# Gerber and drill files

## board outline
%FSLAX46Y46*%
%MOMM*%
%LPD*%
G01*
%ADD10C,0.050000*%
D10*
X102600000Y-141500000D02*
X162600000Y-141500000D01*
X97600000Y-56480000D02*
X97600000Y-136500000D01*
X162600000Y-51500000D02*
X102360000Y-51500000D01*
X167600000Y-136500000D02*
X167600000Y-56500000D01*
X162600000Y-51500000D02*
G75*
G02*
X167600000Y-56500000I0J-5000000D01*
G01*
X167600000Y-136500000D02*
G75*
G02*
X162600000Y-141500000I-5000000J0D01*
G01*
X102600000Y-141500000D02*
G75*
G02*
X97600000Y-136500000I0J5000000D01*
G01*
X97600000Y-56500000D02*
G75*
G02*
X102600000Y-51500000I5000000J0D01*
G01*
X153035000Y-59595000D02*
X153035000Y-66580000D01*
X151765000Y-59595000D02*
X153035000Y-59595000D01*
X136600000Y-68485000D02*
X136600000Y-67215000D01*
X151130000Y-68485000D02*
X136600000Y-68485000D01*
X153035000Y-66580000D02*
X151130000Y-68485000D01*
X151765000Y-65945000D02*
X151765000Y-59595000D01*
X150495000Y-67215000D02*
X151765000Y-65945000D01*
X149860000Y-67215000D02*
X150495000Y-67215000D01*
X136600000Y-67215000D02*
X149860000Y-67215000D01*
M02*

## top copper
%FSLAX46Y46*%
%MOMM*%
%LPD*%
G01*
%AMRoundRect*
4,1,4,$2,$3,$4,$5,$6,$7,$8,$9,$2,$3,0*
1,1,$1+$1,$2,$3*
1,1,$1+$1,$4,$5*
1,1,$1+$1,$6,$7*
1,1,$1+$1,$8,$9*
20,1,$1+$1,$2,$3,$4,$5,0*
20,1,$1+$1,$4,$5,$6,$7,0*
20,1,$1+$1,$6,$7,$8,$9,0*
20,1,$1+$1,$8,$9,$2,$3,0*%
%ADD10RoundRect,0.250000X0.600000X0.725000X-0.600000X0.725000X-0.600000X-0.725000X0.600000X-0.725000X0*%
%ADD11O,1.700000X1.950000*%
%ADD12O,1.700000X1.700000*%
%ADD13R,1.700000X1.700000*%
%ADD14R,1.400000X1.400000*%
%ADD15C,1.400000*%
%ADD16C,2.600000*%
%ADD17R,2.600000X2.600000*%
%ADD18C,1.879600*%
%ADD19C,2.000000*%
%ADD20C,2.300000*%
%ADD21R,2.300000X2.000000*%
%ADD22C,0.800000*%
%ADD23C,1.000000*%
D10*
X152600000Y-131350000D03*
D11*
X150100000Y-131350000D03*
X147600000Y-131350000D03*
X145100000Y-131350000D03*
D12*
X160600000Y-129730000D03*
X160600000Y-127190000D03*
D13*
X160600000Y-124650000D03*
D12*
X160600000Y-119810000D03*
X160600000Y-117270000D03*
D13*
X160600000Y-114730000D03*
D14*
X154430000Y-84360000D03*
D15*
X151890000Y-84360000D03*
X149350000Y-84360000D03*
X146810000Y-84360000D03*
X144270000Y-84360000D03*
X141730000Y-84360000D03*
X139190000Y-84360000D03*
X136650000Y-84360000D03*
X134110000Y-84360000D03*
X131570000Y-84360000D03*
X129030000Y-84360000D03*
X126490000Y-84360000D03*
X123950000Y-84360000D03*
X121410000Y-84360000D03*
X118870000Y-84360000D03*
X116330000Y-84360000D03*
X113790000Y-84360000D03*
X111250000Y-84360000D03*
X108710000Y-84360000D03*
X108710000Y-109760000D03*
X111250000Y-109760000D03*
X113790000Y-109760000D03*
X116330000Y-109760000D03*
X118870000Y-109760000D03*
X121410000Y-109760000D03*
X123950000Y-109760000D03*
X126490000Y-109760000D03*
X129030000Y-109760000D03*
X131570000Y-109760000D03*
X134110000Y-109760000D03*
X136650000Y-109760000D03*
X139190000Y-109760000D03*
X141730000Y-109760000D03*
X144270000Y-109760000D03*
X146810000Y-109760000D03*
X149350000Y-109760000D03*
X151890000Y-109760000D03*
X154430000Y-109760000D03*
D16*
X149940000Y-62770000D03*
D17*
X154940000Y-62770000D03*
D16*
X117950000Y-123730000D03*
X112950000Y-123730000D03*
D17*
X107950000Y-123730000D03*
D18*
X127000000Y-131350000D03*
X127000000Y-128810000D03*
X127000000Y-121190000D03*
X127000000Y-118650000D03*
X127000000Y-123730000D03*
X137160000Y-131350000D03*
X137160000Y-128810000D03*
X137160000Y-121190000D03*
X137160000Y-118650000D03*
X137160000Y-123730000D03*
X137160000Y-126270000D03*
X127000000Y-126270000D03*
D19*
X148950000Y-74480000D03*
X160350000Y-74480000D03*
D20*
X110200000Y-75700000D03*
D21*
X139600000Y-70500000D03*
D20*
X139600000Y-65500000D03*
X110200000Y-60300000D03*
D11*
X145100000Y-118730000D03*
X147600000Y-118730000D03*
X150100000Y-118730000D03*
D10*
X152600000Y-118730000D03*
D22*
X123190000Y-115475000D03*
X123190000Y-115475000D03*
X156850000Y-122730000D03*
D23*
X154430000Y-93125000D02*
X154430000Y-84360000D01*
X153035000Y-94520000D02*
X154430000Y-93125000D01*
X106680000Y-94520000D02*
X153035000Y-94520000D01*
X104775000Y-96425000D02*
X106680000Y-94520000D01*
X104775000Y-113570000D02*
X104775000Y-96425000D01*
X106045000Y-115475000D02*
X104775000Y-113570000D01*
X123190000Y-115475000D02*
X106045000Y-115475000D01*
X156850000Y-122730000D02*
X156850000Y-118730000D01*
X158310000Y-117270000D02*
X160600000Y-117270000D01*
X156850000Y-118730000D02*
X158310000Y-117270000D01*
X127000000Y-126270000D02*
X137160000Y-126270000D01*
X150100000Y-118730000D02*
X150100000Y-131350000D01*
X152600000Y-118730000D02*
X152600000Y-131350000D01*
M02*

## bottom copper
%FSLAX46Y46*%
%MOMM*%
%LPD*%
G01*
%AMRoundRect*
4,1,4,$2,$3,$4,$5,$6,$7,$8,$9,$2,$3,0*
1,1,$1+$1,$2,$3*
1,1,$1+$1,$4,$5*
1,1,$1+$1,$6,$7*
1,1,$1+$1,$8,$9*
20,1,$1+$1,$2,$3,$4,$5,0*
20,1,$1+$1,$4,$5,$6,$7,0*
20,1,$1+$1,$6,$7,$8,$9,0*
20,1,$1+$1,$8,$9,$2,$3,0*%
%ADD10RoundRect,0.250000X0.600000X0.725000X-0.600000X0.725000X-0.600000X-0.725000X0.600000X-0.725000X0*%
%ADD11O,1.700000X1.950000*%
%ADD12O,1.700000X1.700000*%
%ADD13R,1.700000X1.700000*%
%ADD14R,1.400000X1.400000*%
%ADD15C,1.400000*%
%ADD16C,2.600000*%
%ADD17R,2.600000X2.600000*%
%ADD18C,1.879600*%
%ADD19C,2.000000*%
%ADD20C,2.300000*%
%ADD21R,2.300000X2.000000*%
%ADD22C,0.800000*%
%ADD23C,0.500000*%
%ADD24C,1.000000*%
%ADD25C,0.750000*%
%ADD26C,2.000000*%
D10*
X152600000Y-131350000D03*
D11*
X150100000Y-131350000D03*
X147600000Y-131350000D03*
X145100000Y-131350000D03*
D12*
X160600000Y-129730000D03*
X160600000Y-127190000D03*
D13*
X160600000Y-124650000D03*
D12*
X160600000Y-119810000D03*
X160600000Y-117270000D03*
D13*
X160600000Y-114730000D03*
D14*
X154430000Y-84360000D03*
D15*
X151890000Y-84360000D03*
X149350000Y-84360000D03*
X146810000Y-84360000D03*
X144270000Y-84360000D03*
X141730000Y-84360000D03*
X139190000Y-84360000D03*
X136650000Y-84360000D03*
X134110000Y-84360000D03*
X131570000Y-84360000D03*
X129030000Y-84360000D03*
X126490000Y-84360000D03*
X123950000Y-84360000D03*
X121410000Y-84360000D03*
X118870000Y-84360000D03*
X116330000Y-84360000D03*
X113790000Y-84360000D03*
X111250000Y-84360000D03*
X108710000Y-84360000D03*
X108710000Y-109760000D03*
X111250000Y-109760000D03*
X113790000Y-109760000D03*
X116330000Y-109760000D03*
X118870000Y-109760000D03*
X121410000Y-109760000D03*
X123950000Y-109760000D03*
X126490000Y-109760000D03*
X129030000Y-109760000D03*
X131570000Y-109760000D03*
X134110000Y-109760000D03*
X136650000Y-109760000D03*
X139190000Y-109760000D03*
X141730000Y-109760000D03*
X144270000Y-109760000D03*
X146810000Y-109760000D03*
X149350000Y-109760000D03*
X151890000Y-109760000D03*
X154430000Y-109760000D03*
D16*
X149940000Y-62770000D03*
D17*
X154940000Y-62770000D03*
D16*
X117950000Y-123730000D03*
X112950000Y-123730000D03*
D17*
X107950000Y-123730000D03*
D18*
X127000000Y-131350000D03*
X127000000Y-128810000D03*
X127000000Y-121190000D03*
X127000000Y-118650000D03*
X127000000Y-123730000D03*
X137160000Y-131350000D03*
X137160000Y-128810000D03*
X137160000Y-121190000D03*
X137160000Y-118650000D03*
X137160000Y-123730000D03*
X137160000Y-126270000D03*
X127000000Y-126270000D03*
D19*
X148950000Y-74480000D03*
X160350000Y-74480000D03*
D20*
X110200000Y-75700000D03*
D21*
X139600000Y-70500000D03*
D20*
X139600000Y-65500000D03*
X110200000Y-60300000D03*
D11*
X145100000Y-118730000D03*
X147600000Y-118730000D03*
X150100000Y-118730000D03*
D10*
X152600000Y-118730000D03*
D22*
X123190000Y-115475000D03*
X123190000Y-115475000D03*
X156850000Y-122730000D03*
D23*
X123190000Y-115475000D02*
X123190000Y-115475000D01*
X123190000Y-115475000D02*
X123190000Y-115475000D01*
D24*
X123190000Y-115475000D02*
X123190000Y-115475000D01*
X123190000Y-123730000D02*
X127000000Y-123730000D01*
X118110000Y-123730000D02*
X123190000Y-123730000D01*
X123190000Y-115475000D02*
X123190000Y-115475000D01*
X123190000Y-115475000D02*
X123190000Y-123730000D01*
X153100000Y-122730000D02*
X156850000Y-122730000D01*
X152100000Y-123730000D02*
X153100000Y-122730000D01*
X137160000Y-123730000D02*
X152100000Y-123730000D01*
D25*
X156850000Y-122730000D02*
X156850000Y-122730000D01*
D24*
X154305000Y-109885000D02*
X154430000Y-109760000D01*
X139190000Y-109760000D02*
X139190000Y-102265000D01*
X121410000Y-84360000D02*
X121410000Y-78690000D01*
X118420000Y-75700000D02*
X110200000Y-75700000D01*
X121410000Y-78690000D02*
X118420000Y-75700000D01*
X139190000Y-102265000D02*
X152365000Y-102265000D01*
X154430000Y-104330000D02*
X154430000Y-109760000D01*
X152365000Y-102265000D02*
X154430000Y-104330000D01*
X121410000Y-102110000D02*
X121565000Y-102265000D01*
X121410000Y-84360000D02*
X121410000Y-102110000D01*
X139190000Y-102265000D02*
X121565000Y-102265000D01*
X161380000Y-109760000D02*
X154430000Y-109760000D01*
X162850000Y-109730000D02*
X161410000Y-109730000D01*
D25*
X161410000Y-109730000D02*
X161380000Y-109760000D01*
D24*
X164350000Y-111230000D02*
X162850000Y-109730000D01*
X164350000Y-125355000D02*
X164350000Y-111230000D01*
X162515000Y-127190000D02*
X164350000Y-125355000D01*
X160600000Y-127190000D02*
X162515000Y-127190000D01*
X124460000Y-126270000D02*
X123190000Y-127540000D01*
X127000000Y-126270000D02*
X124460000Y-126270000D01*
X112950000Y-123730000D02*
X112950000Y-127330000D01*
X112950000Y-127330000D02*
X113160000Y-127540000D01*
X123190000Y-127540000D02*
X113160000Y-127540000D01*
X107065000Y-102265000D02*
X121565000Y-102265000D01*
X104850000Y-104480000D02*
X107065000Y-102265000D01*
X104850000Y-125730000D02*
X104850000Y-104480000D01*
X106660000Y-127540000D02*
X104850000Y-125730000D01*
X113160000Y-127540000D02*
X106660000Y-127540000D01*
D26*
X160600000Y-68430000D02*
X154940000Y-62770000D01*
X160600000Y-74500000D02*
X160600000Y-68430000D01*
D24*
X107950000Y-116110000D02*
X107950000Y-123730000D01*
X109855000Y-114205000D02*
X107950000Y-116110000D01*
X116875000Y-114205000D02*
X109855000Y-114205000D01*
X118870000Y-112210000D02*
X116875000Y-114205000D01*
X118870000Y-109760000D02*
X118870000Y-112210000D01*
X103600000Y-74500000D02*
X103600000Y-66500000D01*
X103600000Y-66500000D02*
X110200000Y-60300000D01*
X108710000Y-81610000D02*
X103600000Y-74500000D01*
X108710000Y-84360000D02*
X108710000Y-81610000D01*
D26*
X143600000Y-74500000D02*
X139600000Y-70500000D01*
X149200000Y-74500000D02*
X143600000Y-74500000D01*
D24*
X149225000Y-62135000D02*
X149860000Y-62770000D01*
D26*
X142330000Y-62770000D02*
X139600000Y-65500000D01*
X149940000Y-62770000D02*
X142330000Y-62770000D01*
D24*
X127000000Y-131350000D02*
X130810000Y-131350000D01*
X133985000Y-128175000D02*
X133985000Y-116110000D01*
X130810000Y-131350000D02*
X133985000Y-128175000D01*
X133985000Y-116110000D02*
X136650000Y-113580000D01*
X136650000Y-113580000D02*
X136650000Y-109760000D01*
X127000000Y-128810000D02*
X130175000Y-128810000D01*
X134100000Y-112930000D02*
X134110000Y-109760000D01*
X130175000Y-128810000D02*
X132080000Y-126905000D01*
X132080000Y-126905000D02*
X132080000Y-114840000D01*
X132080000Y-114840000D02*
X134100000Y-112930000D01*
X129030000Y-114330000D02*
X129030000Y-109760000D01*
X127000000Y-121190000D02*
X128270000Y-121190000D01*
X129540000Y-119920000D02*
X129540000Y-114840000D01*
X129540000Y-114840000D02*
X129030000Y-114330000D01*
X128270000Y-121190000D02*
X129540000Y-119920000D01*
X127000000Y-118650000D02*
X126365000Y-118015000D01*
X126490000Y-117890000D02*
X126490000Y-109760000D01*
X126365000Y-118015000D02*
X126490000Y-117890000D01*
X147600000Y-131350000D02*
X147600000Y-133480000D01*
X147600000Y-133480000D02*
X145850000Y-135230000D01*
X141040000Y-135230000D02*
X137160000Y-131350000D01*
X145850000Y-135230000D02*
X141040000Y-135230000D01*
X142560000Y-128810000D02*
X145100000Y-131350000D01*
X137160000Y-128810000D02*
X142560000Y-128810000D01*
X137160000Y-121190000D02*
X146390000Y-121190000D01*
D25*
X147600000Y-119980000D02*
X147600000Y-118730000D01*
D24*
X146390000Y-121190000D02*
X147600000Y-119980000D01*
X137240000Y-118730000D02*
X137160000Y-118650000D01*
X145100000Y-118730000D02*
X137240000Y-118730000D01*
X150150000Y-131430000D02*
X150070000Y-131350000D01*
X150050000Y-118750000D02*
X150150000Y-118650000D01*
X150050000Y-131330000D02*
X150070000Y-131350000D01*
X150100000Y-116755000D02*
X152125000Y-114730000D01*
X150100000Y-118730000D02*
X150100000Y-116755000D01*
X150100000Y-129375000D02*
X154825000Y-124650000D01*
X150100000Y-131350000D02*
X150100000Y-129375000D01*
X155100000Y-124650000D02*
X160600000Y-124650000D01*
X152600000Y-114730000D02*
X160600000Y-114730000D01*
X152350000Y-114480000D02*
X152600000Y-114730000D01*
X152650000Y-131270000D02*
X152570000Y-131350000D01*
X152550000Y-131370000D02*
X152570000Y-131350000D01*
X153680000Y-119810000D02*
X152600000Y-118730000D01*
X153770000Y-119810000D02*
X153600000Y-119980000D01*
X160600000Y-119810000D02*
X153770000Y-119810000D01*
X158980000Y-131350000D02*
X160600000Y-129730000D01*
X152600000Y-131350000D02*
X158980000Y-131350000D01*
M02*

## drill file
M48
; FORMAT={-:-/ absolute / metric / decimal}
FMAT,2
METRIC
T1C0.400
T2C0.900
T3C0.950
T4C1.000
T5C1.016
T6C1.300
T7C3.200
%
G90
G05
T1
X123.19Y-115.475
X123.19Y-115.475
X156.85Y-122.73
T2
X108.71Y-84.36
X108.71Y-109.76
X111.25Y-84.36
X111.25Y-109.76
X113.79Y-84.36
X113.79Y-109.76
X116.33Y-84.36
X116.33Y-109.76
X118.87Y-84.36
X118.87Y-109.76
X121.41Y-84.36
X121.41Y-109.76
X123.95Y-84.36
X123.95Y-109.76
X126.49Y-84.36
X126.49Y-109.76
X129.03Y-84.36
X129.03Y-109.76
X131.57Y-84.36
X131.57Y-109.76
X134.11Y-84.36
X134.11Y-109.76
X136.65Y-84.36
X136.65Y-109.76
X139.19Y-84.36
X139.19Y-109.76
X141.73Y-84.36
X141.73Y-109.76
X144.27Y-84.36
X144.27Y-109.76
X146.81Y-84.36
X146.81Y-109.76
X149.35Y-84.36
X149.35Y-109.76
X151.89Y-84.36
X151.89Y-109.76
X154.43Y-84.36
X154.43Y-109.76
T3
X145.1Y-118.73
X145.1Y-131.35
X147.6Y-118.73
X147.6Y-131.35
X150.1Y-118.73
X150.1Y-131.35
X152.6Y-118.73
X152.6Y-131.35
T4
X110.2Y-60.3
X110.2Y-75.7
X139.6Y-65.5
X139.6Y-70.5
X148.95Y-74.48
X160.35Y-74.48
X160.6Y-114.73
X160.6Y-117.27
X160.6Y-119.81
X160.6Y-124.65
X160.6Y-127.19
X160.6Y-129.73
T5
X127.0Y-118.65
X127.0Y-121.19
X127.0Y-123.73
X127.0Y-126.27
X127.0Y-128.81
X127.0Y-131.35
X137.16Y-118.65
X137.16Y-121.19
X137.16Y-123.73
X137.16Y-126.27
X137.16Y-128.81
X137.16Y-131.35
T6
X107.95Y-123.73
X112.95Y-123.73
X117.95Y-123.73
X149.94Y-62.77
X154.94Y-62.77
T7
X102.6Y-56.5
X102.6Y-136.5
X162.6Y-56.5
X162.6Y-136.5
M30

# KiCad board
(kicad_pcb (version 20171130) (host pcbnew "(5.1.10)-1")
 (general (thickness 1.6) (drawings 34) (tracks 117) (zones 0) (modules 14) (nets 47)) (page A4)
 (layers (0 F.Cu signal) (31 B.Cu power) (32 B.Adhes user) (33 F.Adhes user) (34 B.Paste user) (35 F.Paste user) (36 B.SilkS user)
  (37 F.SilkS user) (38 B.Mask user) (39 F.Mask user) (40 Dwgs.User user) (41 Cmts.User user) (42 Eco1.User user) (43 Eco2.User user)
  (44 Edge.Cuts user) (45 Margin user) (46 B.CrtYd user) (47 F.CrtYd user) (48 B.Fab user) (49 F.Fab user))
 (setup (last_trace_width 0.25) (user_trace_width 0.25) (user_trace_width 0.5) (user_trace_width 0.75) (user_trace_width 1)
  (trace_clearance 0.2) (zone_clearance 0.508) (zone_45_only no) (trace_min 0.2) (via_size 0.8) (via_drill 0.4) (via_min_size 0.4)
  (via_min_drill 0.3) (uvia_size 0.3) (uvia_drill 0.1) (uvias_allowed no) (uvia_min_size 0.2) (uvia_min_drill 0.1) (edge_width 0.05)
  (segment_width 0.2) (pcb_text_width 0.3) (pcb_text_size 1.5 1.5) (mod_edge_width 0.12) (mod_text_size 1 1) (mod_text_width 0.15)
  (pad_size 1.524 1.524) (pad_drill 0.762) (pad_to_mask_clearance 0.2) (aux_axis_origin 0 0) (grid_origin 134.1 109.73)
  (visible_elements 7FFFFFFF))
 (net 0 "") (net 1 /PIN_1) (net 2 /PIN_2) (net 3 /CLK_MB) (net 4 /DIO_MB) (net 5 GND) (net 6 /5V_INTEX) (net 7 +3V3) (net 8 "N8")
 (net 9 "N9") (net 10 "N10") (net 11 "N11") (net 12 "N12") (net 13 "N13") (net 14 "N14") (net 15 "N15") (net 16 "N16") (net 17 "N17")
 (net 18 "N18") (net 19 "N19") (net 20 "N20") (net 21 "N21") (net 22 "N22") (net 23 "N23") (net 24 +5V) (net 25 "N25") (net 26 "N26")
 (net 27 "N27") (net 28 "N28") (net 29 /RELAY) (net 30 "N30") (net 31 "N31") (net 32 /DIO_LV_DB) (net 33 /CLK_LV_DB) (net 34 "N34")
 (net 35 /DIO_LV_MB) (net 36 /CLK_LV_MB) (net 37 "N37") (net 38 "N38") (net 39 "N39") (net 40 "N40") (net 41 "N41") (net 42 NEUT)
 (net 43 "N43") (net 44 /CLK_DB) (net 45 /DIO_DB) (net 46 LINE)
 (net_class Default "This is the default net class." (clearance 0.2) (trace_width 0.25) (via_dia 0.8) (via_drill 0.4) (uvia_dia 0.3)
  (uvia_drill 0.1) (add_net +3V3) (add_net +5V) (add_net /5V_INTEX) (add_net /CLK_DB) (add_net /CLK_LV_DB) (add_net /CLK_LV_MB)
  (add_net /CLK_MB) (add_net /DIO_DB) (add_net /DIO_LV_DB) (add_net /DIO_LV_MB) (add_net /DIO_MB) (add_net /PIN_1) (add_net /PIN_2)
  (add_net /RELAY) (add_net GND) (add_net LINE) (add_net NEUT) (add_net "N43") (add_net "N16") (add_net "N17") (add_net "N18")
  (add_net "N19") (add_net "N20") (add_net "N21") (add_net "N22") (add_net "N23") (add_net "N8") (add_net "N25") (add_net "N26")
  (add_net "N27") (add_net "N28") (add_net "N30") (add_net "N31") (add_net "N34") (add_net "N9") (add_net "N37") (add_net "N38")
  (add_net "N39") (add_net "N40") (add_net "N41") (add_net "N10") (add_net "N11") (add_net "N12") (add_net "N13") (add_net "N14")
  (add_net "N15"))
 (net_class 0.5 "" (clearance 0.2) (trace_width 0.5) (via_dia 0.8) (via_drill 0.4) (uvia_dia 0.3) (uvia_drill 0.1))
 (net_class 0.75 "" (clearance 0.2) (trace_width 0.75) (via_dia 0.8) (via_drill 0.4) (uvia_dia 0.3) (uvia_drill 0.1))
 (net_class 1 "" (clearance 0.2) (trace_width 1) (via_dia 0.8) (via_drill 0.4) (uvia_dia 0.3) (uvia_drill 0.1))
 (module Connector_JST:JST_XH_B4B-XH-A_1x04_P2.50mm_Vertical (layer F.Cu) (at 152.6 131.35 180)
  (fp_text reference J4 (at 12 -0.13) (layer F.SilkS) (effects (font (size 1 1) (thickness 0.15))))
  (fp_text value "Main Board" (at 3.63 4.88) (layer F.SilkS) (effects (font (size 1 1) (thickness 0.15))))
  (pad 1 thru_hole roundrect (at 0 0 180) (size 1.7 1.95) (drill 0.95) (layers *.Cu *.Mask) (roundrect_rratio 0.1470588235294118)
   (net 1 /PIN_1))
  (pad 2 thru_hole oval (at 2.5 0 180) (size 1.7 1.95) (drill 0.95) (layers *.Cu *.Mask) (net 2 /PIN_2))
  (pad 3 thru_hole oval (at 5 0 180) (size 1.7 1.95) (drill 0.95) (layers *.Cu *.Mask) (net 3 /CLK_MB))
  (pad 4 thru_hole oval (at 7.5 0 180) (size 1.7 1.95) (drill 0.95) (layers *.Cu *.Mask) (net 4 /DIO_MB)))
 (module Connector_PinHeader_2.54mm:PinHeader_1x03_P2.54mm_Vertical (layer F.Cu) (at 160.6 124.65)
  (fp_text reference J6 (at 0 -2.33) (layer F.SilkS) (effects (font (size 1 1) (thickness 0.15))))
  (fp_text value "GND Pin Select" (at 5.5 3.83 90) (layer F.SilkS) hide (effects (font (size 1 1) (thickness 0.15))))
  (pad 3 thru_hole oval (at 0 5.08) (size 1.7 1.7) (drill 1) (layers *.Cu *.Mask) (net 1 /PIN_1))
  (pad 2 thru_hole oval (at 0 2.54) (size 1.7 1.7) (drill 1) (layers *.Cu *.Mask) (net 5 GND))
  (pad 1 thru_hole rect (at 0 0) (size 1.7 1.7) (drill 1) (layers *.Cu *.Mask) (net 2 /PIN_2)))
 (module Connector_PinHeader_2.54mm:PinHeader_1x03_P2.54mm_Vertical (layer F.Cu) (at 160.6 114.73)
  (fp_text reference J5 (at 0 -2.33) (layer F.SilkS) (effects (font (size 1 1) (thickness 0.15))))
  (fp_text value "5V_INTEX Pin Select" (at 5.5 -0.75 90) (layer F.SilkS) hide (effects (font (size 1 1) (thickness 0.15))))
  (pad 3 thru_hole oval (at 0 5.08) (size 1.7 1.7) (drill 1) (layers *.Cu *.Mask) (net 1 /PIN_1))
  (pad 2 thru_hole oval (at 0 2.54) (size 1.7 1.7) (drill 1) (layers *.Cu *.Mask) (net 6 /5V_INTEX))
  (pad 1 thru_hole rect (at 0 0) (size 1.7 1.7) (drill 1) (layers *.Cu *.Mask) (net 2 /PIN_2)))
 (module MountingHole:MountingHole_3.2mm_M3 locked (layer F.Cu) (at 162.6 136.5)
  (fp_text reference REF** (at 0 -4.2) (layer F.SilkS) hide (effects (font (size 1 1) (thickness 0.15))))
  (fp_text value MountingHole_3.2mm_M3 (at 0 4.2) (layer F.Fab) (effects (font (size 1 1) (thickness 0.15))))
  (pad 1 np_thru_hole circle (at 0 0) (size 3.2 3.2) (drill 3.2) (layers *.Cu *.Mask)))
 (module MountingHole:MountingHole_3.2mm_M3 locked (layer F.Cu) (at 102.6 136.5)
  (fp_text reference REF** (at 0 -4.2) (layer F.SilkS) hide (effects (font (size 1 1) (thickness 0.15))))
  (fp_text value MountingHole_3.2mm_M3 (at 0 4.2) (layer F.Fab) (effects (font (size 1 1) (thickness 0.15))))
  (pad 1 np_thru_hole circle (at 0 0) (size 3.2 3.2) (drill 3.2) (layers *.Cu *.Mask)))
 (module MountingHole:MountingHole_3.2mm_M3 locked (layer F.Cu) (at 162.6 56.5)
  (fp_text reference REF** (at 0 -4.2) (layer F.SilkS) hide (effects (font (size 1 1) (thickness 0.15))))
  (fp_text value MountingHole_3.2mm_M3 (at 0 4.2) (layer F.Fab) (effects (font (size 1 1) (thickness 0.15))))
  (pad 1 np_thru_hole circle (at 0 0) (size 3.2 3.2) (drill 3.2) (layers *.Cu *.Mask)))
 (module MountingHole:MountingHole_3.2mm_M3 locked (layer F.Cu) (at 102.6 56.5)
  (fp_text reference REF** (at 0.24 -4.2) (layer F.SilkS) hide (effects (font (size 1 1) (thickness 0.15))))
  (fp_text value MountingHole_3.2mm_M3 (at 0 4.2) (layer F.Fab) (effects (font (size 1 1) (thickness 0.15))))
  (pad 1 np_thru_hole circle (at 0 0) (size 3.2 3.2) (drill 3.2) (layers *.Cu *.Mask)))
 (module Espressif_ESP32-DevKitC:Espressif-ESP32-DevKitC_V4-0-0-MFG (layer F.Cu) (at 134.62 97.06 270)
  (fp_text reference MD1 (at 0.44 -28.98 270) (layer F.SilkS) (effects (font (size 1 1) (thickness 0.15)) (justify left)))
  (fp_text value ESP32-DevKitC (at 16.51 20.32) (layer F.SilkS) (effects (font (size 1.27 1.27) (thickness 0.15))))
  (pad 1 thru_hole rect (at -12.7 -19.81 270) (size 1.4 1.4) (drill 0.9) (layers *.Cu *.Paste *.Mask) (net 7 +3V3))
  (pad 2 thru_hole circle (at -12.7 -17.27 270) (size 1.4 1.4) (drill 0.9) (layers *.Cu *.Paste *.Mask) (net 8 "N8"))
  (pad 3 thru_hole circle (at -12.7 -14.73 270) (size 1.4 1.4) (drill 0.9) (layers *.Cu *.Paste *.Mask) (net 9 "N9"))
  (pad 4 thru_hole circle (at -12.7 -12.19 270) (size 1.4 1.4) (drill 0.9) (layers *.Cu *.Paste *.Mask) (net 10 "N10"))
  (pad 5 thru_hole circle (at -12.7 -9.65 270) (size 1.4 1.4) (drill 0.9) (layers *.Cu *.Paste *.Mask) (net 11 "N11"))
  (pad 6 thru_hole circle (at -12.7 -7.11 270) (size 1.4 1.4) (drill 0.9) (layers *.Cu *.Paste *.Mask) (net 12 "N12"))
  (pad 7 thru_hole circle (at -12.7 -4.57 270) (size 1.4 1.4) (drill 0.9) (layers *.Cu *.Paste *.Mask) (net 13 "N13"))
  (pad 8 thru_hole circle (at -12.7 -2.03 270) (size 1.4 1.4) (drill 0.9) (layers *.Cu *.Paste *.Mask) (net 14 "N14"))
  (pad 9 thru_hole circle (at -12.7 0.51 270) (size 1.4 1.4) (drill 0.9) (layers *.Cu *.Paste *.Mask) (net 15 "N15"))
  (pad 10 thru_hole circle (at -12.7 3.05 270) (size 1.4 1.4) (drill 0.9) (layers *.Cu *.Paste *.Mask) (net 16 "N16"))
  (pad 11 thru_hole circle (at -12.7 5.59 270) (size 1.4 1.4) (drill 0.9) (layers *.Cu *.Paste *.Mask) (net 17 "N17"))
  (pad 12 thru_hole circle (at -12.7 8.13 270) (size 1.4 1.4) (drill 0.9) (layers *.Cu *.Paste *.Mask) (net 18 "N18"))
  (pad 13 thru_hole circle (at -12.7 10.67 270) (size 1.4 1.4) (drill 0.9) (layers *.Cu *.Paste *.Mask) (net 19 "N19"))
  (pad 14 thru_hole circle (at -12.7 13.21 270) (size 1.4 1.4) (drill 0.9) (layers *.Cu *.Paste *.Mask) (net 5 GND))
  (pad 15 thru_hole circle (at -12.7 15.75 270) (size 1.4 1.4) (drill 0.9) (layers *.Cu *.Paste *.Mask) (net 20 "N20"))
  (pad 16 thru_hole circle (at -12.7 18.29 270) (size 1.4 1.4) (drill 0.9) (layers *.Cu *.Paste *.Mask) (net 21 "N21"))
  (pad 17 thru_hole circle (at -12.7 20.83 270) (size 1.4 1.4) (drill 0.9) (layers *.Cu *.Paste *.Mask) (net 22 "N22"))
  (pad 18 thru_hole circle (at -12.7 23.37 270) (size 1.4 1.4) (drill 0.9) (layers *.Cu *.Paste *.Mask) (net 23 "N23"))
  (pad 19 thru_hole circle (at -12.7 25.91 270) (size 1.4 1.4) (drill 0.9) (layers *.Cu *.Paste *.Mask) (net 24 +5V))
  (pad 20 thru_hole circle (at 12.7 25.91 270) (size 1.4 1.4) (drill 0.9) (layers *.Cu *.Paste *.Mask) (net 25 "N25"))
  (pad 21 thru_hole circle (at 12.7 23.37 270) (size 1.4 1.4) (drill 0.9) (layers *.Cu *.Paste *.Mask) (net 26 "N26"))
  (pad 22 thru_hole circle (at 12.7 20.83 270) (size 1.4 1.4) (drill 0.9) (layers *.Cu *.Paste *.Mask) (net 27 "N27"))
  (pad 23 thru_hole circle (at 12.7 18.29 270) (size 1.4 1.4) (drill 0.9) (layers *.Cu *.Paste *.Mask) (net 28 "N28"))
  (pad 24 thru_hole circle (at 12.7 15.75 270) (size 1.4 1.4) (drill 0.9) (layers *.Cu *.Paste *.Mask) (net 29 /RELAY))
  (pad 25 thru_hole circle (at 12.7 13.21 270) (size 1.4 1.4) (drill 0.9) (layers *.Cu *.Paste *.Mask) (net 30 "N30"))
  (pad 26 thru_hole circle (at 12.7 10.67 270) (size 1.4 1.4) (drill 0.9) (layers *.Cu *.Paste *.Mask) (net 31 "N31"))
  (pad 27 thru_hole circle (at 12.7 8.13 270) (size 1.4 1.4) (drill 0.9) (layers *.Cu *.Paste *.Mask) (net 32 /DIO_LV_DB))
  (pad 28 thru_hole circle (at 12.7 5.59 270) (size 1.4 1.4) (drill 0.9) (layers *.Cu *.Paste *.Mask) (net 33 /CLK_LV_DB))
  (pad 29 thru_hole circle (at 12.7 3.05 270) (size 1.4 1.4) (drill 0.9) (layers *.Cu *.Paste *.Mask) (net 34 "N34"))
  (pad 30 thru_hole circle (at 12.7 0.51 270) (size 1.4 1.4) (drill 0.9) (layers *.Cu *.Paste *.Mask) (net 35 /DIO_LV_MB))
  (pad 31 thru_hole circle (at 12.7 -2.03 270) (size 1.4 1.4) (drill 0.9) (layers *.Cu *.Paste *.Mask) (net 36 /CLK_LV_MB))
  (pad 32 thru_hole circle (at 12.7 -4.57 270) (size 1.4 1.4) (drill 0.9) (layers *.Cu *.Paste *.Mask) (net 5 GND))
  (pad 33 thru_hole circle (at 12.7 -7.11 270) (size 1.4 1.4) (drill 0.9) (layers *.Cu *.Paste *.Mask) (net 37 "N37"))
  (pad 34 thru_hole circle (at 12.7 -9.65 270) (size 1.4 1.4) (drill 0.9) (layers *.Cu *.Paste *.Mask) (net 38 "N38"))
  (pad 35 thru_hole circle (at 12.7 -12.19 270) (size 1.4 1.4) (drill 0.9) (layers *.Cu *.Paste *.Mask) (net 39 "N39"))
  (pad 36 thru_hole circle (at 12.7 -14.73 270) (size 1.4 1.4) (drill 0.9) (layers *.Cu *.Paste *.Mask) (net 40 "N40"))
  (pad 37 thru_hole circle (at 12.7 -17.27 270) (size 1.4 1.4) (drill 0.9) (layers *.Cu *.Paste *.Mask) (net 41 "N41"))
  (pad 38 thru_hole circle (at 12.7 -19.81 270) (size 1.4 1.4) (drill 0.9) (layers *.Cu *.Paste *.Mask) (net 5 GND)))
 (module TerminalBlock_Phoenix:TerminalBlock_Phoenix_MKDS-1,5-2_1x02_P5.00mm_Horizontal (layer F.Cu) (at 154.94 62.77 180)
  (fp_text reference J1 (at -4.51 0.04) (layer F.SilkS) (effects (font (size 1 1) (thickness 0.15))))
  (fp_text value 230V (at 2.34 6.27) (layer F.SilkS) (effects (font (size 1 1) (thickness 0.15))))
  (pad 2 thru_hole circle (at 5 0 180) (size 2.6 2.6) (drill 1.3) (layers *.Cu *.Mask) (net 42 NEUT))
  (pad 1 thru_hole rect (at 0 0 180) (size 2.6 2.6) (drill 1.3) (layers *.Cu *.Mask) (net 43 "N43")))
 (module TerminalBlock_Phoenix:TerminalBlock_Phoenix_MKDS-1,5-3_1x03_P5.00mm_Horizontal (layer F.Cu) (at 107.95 123.73)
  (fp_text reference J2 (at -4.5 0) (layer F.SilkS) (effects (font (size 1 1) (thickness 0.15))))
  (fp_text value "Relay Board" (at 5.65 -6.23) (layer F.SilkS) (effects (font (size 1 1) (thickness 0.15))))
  (pad 3 thru_hole circle (at 10 0) (size 2.6 2.6) (drill 1.3) (layers *.Cu *.Mask) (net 7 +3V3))
  (pad 2 thru_hole circle (at 5 0) (size 2.6 2.6) (drill 1.3) (layers *.Cu *.Mask) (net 5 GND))
  (pad 1 thru_hole rect (at 0 0) (size 2.6 2.6) (drill 1.3) (layers *.Cu *.Mask) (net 29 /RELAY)))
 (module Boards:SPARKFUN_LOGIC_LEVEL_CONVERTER (layer F.Cu) (at 132.08 125)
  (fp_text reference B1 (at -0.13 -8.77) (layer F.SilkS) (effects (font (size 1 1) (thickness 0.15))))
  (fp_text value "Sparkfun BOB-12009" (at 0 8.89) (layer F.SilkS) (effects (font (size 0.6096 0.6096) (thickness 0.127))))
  (pad LV4 thru_hole circle (at -5.08 6.35) (size 1.8796 1.8796) (drill 1.016) (layers *.Cu *.Mask) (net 36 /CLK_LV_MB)
   (solder_mask_margin 0.1016))
  (pad LV3 thru_hole circle (at -5.08 3.81) (size 1.8796 1.8796) (drill 1.016) (layers *.Cu *.Mask) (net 35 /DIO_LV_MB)
   (solder_mask_margin 0.1016))
  (pad LV2 thru_hole circle (at -5.08 -3.81) (size 1.8796 1.8796) (drill 1.016) (layers *.Cu *.Mask) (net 33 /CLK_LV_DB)
   (solder_mask_margin 0.1016))
  (pad LV1 thru_hole circle (at -5.08 -6.35) (size 1.8796 1.8796) (drill 1.016) (layers *.Cu *.Mask) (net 32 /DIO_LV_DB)
   (solder_mask_margin 0.1016))
  (pad LV thru_hole circle (at -5.08 -1.27) (size 1.8796 1.8796) (drill 1.016) (layers *.Cu *.Mask) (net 7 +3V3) (solder_mask_margin 0.1016))
  (pad HV4 thru_hole circle (at 5.08 6.35) (size 1.8796 1.8796) (drill 1.016) (layers *.Cu *.Mask) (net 3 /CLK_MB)
   (solder_mask_margin 0.1016))
  (pad HV3 thru_hole circle (at 5.08 3.81) (size 1.8796 1.8796) (drill 1.016) (layers *.Cu *.Mask) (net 4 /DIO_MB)
   (solder_mask_margin 0.1016))
  (pad HV2 thru_hole circle (at 5.08 -3.81) (size 1.8796 1.8796) (drill 1.016) (layers *.Cu *.Mask) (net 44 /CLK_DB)
   (solder_mask_margin 0.1016))
  (pad HV1 thru_hole circle (at 5.08 -6.35) (size 1.8796 1.8796) (drill 1.016) (layers *.Cu *.Mask) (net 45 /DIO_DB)
   (solder_mask_margin 0.1016))
  (pad HV thru_hole circle (at 5.08 -1.27) (size 1.8796 1.8796) (drill 1.016) (layers *.Cu *.Mask) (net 6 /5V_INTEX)
   (solder_mask_margin 0.1016))
  (pad GND2 thru_hole circle (at 5.08 1.27) (size 1.8796 1.8796) (drill 1.016) (layers *.Cu *.Mask) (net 5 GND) (solder_mask_margin 0.1016))
  (pad GND1 thru_hole circle (at -5.08 1.27) (size 1.8796 1.8796) (drill 1.016) (layers *.Cu *.Mask) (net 5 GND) (solder_mask_margin 0.1016)))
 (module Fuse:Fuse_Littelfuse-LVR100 (layer F.Cu) (at 160.35 74.48 180)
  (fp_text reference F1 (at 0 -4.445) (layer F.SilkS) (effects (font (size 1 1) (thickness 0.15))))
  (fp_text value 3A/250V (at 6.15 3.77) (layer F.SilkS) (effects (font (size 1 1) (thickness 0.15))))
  (pad 2 thru_hole circle (at 11.4 0 180) (size 2 2) (drill 1) (layers *.Cu *.Mask) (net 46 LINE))
  (pad 1 thru_hole circle (at 0 0 180) (size 2 2) (drill 1) (layers *.Cu *.Mask) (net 43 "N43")))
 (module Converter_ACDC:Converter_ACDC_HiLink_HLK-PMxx (layer F.Cu) (at 139.6 70.5 180)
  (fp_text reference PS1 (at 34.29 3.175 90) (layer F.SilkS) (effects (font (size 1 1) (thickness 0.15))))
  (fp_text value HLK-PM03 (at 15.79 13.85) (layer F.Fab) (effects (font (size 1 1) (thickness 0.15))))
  (pad 3 thru_hole circle (at 29.4 -5.2 180) (size 2.3 2.3) (drill 1) (layers *.Cu *.Mask) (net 5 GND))
  (pad 1 thru_hole rect (at 0 0 180) (size 2.3 2) (drill 1) (layers *.Cu *.Mask) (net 46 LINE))
  (pad 2 thru_hole circle (at 0 5 180) (size 2.3 2.3) (drill 1) (layers *.Cu *.Mask) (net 42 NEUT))
  (pad 4 thru_hole circle (at 29.4 10.2 180) (size 2.3 2.3) (drill 1) (layers *.Cu *.Mask) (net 24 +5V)))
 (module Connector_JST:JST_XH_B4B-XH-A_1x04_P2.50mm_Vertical (layer F.Cu) (at 152.6 118.73 180)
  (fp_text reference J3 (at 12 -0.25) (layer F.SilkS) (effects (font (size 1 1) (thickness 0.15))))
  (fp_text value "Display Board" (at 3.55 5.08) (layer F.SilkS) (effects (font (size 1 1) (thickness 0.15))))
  (pad 4 thru_hole oval (at 7.5 0 180) (size 1.7 1.95) (drill 0.95) (layers *.Cu *.Mask) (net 45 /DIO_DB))
  (pad 3 thru_hole oval (at 5 0 180) (size 1.7 1.95) (drill 0.95) (layers *.Cu *.Mask) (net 44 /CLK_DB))
  (pad 2 thru_hole oval (at 2.5 0 180) (size 1.7 1.95) (drill 0.95) (layers *.Cu *.Mask) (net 2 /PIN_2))
  (pad 1 thru_hole roundrect (at 0 0 180) (size 1.7 1.95) (drill 0.95) (layers *.Cu *.Mask) (roundrect_rratio 0.1470588235294118)
   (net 1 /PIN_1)))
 (gr_line (start 102.6 141.5) (end 162.6 141.5) (layer Edge.Cuts) (width 0.05))
 (gr_line (start 97.6 56.48) (end 97.6 136.5) (layer Edge.Cuts) (width 0.05))
 (gr_line (start 162.6 51.5) (end 102.36 51.5) (layer Edge.Cuts) (width 0.05))
 (gr_line (start 167.6 136.5) (end 167.6 56.5) (layer Edge.Cuts) (width 0.05))
 (gr_arc (start 162.6 56.5) (end 167.6 56.5) (angle -90) (layer Edge.Cuts) (width 0.05))
 (gr_arc (start 162.6 136.5) (end 162.6 141.5) (angle -90) (layer Edge.Cuts) (width 0.05))
 (gr_arc (start 102.6 136.5) (end 97.6 136.5) (angle -90) (layer Edge.Cuts) (width 0.05))
 (gr_arc (start 102.6 56.5) (end 102.6 51.5) (angle -90) (layer Edge.Cuts) (width 0.05))
 (gr_line (start 153.035 59.595) (end 153.035 66.58) (layer Edge.Cuts) (width 0.05))
 (gr_line (start 151.765 59.595) (end 153.035 59.595) (layer Edge.Cuts) (width 0.05))
 (gr_line (start 136.6 68.485) (end 136.6 67.215) (layer Edge.Cuts) (width 0.05))
 (gr_line (start 151.13 68.485) (end 136.6 68.485) (layer Edge.Cuts) (width 0.05))
 (gr_line (start 153.035 66.58) (end 151.13 68.485) (layer Edge.Cuts) (width 0.05))
 (gr_line (start 151.765 65.945) (end 151.765 59.595) (layer Edge.Cuts) (width 0.05))
 (gr_line (start 150.495 67.215) (end 151.765 65.945) (layer Edge.Cuts) (width 0.05))
 (gr_line (start 149.86 67.215) (end 150.495 67.215) (layer Edge.Cuts) (width 0.05))
 (gr_line (start 136.6 67.215) (end 149.86 67.215) (layer Edge.Cuts) (width 0.05))
 (segment (start 123.19 115.475) (end 123.19 115.475) (width 0.5) (layer B.Cu) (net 7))
 (segment (start 123.19 115.475) (end 123.19 115.475) (width 0.5) (layer B.Cu) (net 7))
 (segment (start 123.19 115.475) (end 123.19 115.475) (width 1) (layer B.Cu) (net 7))
 (segment (start 123.19 123.73) (end 127 123.73) (width 1) (layer B.Cu) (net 7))
 (segment (start 118.11 123.73) (end 123.19 123.73) (width 1) (layer B.Cu) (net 7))
 (segment (start 123.19 115.475) (end 123.19 115.475) (width 1) (layer B.Cu) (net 7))
 (via (at 123.19 115.475) (size 0.8) (drill 0.4) (layers F.Cu B.Cu) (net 7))
 (segment (start 123.19 115.475) (end 123.19 123.73) (width 1) (layer B.Cu) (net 7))
 (via (at 123.19 115.475) (size 0.8) (drill 0.4) (layers F.Cu B.Cu) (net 7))
 (segment (start 154.43 93.125) (end 154.43 84.36) (width 1) (layer F.Cu) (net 7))
 (segment (start 153.035 94.52) (end 154.43 93.125) (width 1) (layer F.Cu) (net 7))
 (segment (start 106.68 94.52) (end 153.035 94.52) (width 1) (layer F.Cu) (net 7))
 (segment (start 104.775 96.425) (end 106.68 94.52) (width 1) (layer F.Cu) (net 7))
 (segment (start 104.775 113.57) (end 104.775 96.425) (width 1) (layer F.Cu) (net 7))
 (segment (start 106.045 115.475) (end 104.775 113.57) (width 1) (layer F.Cu) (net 7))
 (segment (start 123.19 115.475) (end 106.045 115.475) (width 1) (layer F.Cu) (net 7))
 (segment (start 153.1 122.73) (end 156.85 122.73) (width 1) (layer B.Cu) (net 6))
 (segment (start 152.1 123.73) (end 153.1 122.73) (width 1) (layer B.Cu) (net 6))
 (segment (start 137.16 123.73) (end 152.1 123.73) (width 1) (layer B.Cu) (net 6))
 (segment (start 156.85 122.73) (end 156.85 122.73) (width 0.75) (layer B.Cu) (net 6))
 (via (at 156.85 122.73) (size 0.8) (drill 0.4) (layers F.Cu B.Cu) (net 6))
 (segment (start 156.85 122.73) (end 156.85 118.73) (width 1) (layer F.Cu) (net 6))
 (segment (start 158.31 117.27) (end 160.6 117.27) (width 1) (layer F.Cu) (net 6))
 (segment (start 156.85 118.73) (end 158.31 117.27) (width 1) (layer F.Cu) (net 6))
 (segment (start 154.305 109.885) (end 154.43 109.76) (width 1) (layer B.Cu) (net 5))
 (segment (start 139.19 109.76) (end 139.19 102.265) (width 1) (layer B.Cu) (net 5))
 (segment (start 121.41 84.36) (end 121.41 78.69) (width 1) (layer B.Cu) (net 5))
 (segment (start 118.42 75.7) (end 110.2 75.7) (width 1) (layer B.Cu) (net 5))
 (segment (start 121.41 78.69) (end 118.42 75.7) (width 1) (layer B.Cu) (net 5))
 (segment (start 139.19 102.265) (end 152.365 102.265) (width 1) (layer B.Cu) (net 5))
 (segment (start 154.43 104.33) (end 154.43 109.76) (width 1) (layer B.Cu) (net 5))
 (segment (start 152.365 102.265) (end 154.43 104.33) (width 1) (layer B.Cu) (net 5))
 (segment (start 121.41 102.11) (end 121.565 102.265) (width 1) (layer B.Cu) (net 5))
 (segment (start 121.41 84.36) (end 121.41 102.11) (width 1) (layer B.Cu) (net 5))
 (segment (start 139.19 102.265) (end 121.565 102.265) (width 1) (layer B.Cu) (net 5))
 (segment (start 127 126.27) (end 137.16 126.27) (width 1) (layer F.Cu) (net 5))
 (segment (start 161.38 109.76) (end 154.43 109.76) (width 1) (layer B.Cu) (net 5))
 (segment (start 162.85 109.73) (end 161.41 109.73) (width 1) (layer B.Cu) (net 5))
 (segment (start 161.41 109.73) (end 161.38 109.76) (width 0.75) (layer B.Cu) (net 5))
 (segment (start 164.35 111.23) (end 162.85 109.73) (width 1) (layer B.Cu) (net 5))
 (segment (start 164.35 125.355) (end 164.35 111.23) (width 1) (layer B.Cu) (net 5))
 (segment (start 162.515 127.19) (end 164.35 125.355) (width 1) (layer B.Cu) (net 5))
 (segment (start 160.6 127.19) (end 162.515 127.19) (width 1) (layer B.Cu) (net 5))
 (segment (start 124.46 126.27) (end 123.19 127.54) (width 1) (layer B.Cu) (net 5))
 (segment (start 127 126.27) (end 124.46 126.27) (width 1) (layer B.Cu) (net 5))
 (segment (start 112.95 123.73) (end 112.95 127.33) (width 1) (layer B.Cu) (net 5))
 (segment (start 112.95 127.33) (end 113.16 127.54) (width 1) (layer B.Cu) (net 5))
 (segment (start 123.19 127.54) (end 113.16 127.54) (width 1) (layer B.Cu) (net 5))
 (segment (start 107.065 102.265) (end 121.565 102.265) (width 1) (layer B.Cu) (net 5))
 (segment (start 104.85 104.48) (end 107.065 102.265) (width 1) (layer B.Cu) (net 5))
 (segment (start 104.85 125.73) (end 104.85 104.48) (width 1) (layer B.Cu) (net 5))
 (segment (start 106.66 127.54) (end 104.85 125.73) (width 1) (layer B.Cu) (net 5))
 (segment (start 113.16 127.54) (end 106.66 127.54) (width 1) (layer B.Cu) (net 5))
 (segment (start 160.6 68.43) (end 154.94 62.77) (width 2) (layer B.Cu) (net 43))
 (segment (start 160.6 74.5) (end 160.6 68.43) (width 2) (layer B.Cu) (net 43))
 (segment (start 107.95 116.11) (end 107.95 123.73) (width 1) (layer B.Cu) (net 29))
 (segment (start 109.855 114.205) (end 107.95 116.11) (width 1) (layer B.Cu) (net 29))
 (segment (start 116.875 114.205) (end 109.855 114.205) (width 1) (layer B.Cu) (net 29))
 (segment (start 118.87 112.21) (end 116.875 114.205) (width 1) (layer B.Cu) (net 29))
 (segment (start 118.87 109.76) (end 118.87 112.21) (width 1) (layer B.Cu) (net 29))
 (segment (start 103.6 74.5) (end 103.6 66.5) (width 1) (layer B.Cu) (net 24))
 (segment (start 103.6 66.5) (end 110.2 60.3) (width 1) (layer B.Cu) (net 24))
 (segment (start 108.71 81.61) (end 103.6 74.5) (width 1) (layer B.Cu) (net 24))
 (segment (start 108.71 84.36) (end 108.71 81.61) (width 1) (layer B.Cu) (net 24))
 (segment (start 143.6 74.5) (end 139.6 70.5) (width 2) (layer B.Cu) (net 46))
 (segment (start 149.2 74.5) (end 143.6 74.5) (width 2) (layer B.Cu) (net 46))
 (segment (start 149.225 62.135) (end 149.86 62.77) (width 1) (layer B.Cu) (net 42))
 (segment (start 142.33 62.77) (end 139.6 65.5) (width 2) (layer B.Cu) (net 42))
 (segment (start 149.94 62.77) (end 142.33 62.77) (width 2) (layer B.Cu) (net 42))
 (segment (start 127 131.35) (end 130.81 131.35) (width 1) (layer B.Cu) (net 36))
 (segment (start 133.985 128.175) (end 133.985 116.11) (width 1) (layer B.Cu) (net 36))
 (segment (start 130.81 131.35) (end 133.985 128.175) (width 1) (layer B.Cu) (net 36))
 (segment (start 133.985 116.11) (end 136.65 113.58) (width 1) (layer B.Cu) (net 36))
 (segment (start 136.65 113.58) (end 136.65 109.76) (width 1) (layer B.Cu) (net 36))
 (segment (start 127 128.81) (end 130.175 128.81) (width 1) (layer B.Cu) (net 35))
 (segment (start 134.1 112.93) (end 134.11 109.76) (width 1) (layer B.Cu) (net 35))
 (segment (start 130.175 128.81) (end 132.08 126.905) (width 1) (layer B.Cu) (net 35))
 (segment (start 132.08 126.905) (end 132.08 114.84) (width 1) (layer B.Cu) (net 35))
 (segment (start 132.08 114.84) (end 134.1 112.93) (width 1) (layer B.Cu) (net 35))
 (segment (start 129.03 114.33) (end 129.03 109.76) (width 1) (layer B.Cu) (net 33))
 (segment (start 127 121.19) (end 128.27 121.19) (width 1) (layer B.Cu) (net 33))
 (segment (start 129.54 119.92) (end 129.54 114.84) (width 1) (layer B.Cu) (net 33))
 (segment (start 129.54 114.84) (end 129.03 114.33) (width 1) (layer B.Cu) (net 33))
 (segment (start 128.27 121.19) (end 129.54 119.92) (width 1) (layer B.Cu) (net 33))
 (segment (start 127 118.65) (end 126.365 118.015) (width 1) (layer B.Cu) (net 32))
 (segment (start 126.49 117.89) (end 126.49 109.76) (width 1) (layer B.Cu) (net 32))
 (segment (start 126.365 118.015) (end 126.49 117.89) (width 1) (layer B.Cu) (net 32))
 (segment (start 147.6 131.35) (end 147.6 133.48) (width 1) (layer B.Cu) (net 3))
 (segment (start 147.6 133.48) (end 145.85 135.23) (width 1) (layer B.Cu) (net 3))
 (segment (start 141.04 135.23) (end 137.16 131.35) (width 1) (layer B.Cu) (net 3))
 (segment (start 145.85 135.23) (end 141.04 135.23) (width 1) (layer B.Cu) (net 3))
 (segment (start 142.56 128.81) (end 145.1 131.35) (width 1) (layer B.Cu) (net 4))
 (segment (start 137.16 128.81) (end 142.56 128.81) (width 1) (layer B.Cu) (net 4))
 (segment (start 137.16 121.19) (end 146.39 121.19) (width 1) (layer B.Cu) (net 44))
 (segment (start 147.6 119.98) (end 147.6 118.73) (width 0.75) (layer B.Cu) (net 44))
 (segment (start 146.39 121.19) (end 147.6 119.98) (width 1) (layer B.Cu) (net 44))
 (segment (start 137.24 118.73) (end 137.16 118.65) (width 1) (layer B.Cu) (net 45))
 (segment (start 145.1 118.73) (end 137.24 118.73) (width 1) (layer B.Cu) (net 45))
 (segment (start 150.15 131.43) (end 150.07 131.35) (width 1) (layer B.Cu) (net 2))
 (segment (start 150.05 118.75) (end 150.15 118.65) (width 1) (layer B.Cu) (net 2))
 (segment (start 150.05 131.33) (end 150.07 131.35) (width 1) (layer B.Cu) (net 2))
 (segment (start 150.1 118.73) (end 150.1 131.35) (width 1) (layer F.Cu) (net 2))
 (segment (start 150.1 116.755) (end 152.125 114.73) (width 1) (layer B.Cu) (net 2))
 (segment (start 150.1 118.73) (end 150.1 116.755) (width 1) (layer B.Cu) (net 2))
 (segment (start 150.1 129.375) (end 154.825 124.65) (width 1) (layer B.Cu) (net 2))
 (segment (start 150.1 131.35) (end 150.1 129.375) (width 1) (layer B.Cu) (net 2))
 (segment (start 155.1 124.65) (end 160.6 124.65) (width 1) (layer B.Cu) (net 2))
 (segment (start 152.6 114.73) (end 160.6 114.73) (width 1) (layer B.Cu) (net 2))
 (segment (start 152.35 114.48) (end 152.6 114.73) (width 1) (layer B.Cu) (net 2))
 (segment (start 152.65 131.27) (end 152.57 131.35) (width 1) (layer B.Cu) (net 1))
 (segment (start 152.55 131.37) (end 152.57 131.35) (width 1) (layer B.Cu) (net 1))
 (segment (start 152.6 118.73) (end 152.6 131.35) (width 1) (layer F.Cu) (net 1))
 (segment (start 153.68 119.81) (end 152.6 118.73) (width 1) (layer B.Cu) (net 1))
 (segment (start 153.77 119.81) (end 153.6 119.98) (width 1) (layer B.Cu) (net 1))
 (segment (start 160.6 119.81) (end 153.77 119.81) (width 1) (layer B.Cu) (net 1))
 (segment (start 158.98 131.35) (end 160.6 129.73) (width 1) (layer B.Cu) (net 1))
 (segment (start 152.6 131.35) (end 158.98 131.35) (width 1) (layer B.Cu) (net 1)))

